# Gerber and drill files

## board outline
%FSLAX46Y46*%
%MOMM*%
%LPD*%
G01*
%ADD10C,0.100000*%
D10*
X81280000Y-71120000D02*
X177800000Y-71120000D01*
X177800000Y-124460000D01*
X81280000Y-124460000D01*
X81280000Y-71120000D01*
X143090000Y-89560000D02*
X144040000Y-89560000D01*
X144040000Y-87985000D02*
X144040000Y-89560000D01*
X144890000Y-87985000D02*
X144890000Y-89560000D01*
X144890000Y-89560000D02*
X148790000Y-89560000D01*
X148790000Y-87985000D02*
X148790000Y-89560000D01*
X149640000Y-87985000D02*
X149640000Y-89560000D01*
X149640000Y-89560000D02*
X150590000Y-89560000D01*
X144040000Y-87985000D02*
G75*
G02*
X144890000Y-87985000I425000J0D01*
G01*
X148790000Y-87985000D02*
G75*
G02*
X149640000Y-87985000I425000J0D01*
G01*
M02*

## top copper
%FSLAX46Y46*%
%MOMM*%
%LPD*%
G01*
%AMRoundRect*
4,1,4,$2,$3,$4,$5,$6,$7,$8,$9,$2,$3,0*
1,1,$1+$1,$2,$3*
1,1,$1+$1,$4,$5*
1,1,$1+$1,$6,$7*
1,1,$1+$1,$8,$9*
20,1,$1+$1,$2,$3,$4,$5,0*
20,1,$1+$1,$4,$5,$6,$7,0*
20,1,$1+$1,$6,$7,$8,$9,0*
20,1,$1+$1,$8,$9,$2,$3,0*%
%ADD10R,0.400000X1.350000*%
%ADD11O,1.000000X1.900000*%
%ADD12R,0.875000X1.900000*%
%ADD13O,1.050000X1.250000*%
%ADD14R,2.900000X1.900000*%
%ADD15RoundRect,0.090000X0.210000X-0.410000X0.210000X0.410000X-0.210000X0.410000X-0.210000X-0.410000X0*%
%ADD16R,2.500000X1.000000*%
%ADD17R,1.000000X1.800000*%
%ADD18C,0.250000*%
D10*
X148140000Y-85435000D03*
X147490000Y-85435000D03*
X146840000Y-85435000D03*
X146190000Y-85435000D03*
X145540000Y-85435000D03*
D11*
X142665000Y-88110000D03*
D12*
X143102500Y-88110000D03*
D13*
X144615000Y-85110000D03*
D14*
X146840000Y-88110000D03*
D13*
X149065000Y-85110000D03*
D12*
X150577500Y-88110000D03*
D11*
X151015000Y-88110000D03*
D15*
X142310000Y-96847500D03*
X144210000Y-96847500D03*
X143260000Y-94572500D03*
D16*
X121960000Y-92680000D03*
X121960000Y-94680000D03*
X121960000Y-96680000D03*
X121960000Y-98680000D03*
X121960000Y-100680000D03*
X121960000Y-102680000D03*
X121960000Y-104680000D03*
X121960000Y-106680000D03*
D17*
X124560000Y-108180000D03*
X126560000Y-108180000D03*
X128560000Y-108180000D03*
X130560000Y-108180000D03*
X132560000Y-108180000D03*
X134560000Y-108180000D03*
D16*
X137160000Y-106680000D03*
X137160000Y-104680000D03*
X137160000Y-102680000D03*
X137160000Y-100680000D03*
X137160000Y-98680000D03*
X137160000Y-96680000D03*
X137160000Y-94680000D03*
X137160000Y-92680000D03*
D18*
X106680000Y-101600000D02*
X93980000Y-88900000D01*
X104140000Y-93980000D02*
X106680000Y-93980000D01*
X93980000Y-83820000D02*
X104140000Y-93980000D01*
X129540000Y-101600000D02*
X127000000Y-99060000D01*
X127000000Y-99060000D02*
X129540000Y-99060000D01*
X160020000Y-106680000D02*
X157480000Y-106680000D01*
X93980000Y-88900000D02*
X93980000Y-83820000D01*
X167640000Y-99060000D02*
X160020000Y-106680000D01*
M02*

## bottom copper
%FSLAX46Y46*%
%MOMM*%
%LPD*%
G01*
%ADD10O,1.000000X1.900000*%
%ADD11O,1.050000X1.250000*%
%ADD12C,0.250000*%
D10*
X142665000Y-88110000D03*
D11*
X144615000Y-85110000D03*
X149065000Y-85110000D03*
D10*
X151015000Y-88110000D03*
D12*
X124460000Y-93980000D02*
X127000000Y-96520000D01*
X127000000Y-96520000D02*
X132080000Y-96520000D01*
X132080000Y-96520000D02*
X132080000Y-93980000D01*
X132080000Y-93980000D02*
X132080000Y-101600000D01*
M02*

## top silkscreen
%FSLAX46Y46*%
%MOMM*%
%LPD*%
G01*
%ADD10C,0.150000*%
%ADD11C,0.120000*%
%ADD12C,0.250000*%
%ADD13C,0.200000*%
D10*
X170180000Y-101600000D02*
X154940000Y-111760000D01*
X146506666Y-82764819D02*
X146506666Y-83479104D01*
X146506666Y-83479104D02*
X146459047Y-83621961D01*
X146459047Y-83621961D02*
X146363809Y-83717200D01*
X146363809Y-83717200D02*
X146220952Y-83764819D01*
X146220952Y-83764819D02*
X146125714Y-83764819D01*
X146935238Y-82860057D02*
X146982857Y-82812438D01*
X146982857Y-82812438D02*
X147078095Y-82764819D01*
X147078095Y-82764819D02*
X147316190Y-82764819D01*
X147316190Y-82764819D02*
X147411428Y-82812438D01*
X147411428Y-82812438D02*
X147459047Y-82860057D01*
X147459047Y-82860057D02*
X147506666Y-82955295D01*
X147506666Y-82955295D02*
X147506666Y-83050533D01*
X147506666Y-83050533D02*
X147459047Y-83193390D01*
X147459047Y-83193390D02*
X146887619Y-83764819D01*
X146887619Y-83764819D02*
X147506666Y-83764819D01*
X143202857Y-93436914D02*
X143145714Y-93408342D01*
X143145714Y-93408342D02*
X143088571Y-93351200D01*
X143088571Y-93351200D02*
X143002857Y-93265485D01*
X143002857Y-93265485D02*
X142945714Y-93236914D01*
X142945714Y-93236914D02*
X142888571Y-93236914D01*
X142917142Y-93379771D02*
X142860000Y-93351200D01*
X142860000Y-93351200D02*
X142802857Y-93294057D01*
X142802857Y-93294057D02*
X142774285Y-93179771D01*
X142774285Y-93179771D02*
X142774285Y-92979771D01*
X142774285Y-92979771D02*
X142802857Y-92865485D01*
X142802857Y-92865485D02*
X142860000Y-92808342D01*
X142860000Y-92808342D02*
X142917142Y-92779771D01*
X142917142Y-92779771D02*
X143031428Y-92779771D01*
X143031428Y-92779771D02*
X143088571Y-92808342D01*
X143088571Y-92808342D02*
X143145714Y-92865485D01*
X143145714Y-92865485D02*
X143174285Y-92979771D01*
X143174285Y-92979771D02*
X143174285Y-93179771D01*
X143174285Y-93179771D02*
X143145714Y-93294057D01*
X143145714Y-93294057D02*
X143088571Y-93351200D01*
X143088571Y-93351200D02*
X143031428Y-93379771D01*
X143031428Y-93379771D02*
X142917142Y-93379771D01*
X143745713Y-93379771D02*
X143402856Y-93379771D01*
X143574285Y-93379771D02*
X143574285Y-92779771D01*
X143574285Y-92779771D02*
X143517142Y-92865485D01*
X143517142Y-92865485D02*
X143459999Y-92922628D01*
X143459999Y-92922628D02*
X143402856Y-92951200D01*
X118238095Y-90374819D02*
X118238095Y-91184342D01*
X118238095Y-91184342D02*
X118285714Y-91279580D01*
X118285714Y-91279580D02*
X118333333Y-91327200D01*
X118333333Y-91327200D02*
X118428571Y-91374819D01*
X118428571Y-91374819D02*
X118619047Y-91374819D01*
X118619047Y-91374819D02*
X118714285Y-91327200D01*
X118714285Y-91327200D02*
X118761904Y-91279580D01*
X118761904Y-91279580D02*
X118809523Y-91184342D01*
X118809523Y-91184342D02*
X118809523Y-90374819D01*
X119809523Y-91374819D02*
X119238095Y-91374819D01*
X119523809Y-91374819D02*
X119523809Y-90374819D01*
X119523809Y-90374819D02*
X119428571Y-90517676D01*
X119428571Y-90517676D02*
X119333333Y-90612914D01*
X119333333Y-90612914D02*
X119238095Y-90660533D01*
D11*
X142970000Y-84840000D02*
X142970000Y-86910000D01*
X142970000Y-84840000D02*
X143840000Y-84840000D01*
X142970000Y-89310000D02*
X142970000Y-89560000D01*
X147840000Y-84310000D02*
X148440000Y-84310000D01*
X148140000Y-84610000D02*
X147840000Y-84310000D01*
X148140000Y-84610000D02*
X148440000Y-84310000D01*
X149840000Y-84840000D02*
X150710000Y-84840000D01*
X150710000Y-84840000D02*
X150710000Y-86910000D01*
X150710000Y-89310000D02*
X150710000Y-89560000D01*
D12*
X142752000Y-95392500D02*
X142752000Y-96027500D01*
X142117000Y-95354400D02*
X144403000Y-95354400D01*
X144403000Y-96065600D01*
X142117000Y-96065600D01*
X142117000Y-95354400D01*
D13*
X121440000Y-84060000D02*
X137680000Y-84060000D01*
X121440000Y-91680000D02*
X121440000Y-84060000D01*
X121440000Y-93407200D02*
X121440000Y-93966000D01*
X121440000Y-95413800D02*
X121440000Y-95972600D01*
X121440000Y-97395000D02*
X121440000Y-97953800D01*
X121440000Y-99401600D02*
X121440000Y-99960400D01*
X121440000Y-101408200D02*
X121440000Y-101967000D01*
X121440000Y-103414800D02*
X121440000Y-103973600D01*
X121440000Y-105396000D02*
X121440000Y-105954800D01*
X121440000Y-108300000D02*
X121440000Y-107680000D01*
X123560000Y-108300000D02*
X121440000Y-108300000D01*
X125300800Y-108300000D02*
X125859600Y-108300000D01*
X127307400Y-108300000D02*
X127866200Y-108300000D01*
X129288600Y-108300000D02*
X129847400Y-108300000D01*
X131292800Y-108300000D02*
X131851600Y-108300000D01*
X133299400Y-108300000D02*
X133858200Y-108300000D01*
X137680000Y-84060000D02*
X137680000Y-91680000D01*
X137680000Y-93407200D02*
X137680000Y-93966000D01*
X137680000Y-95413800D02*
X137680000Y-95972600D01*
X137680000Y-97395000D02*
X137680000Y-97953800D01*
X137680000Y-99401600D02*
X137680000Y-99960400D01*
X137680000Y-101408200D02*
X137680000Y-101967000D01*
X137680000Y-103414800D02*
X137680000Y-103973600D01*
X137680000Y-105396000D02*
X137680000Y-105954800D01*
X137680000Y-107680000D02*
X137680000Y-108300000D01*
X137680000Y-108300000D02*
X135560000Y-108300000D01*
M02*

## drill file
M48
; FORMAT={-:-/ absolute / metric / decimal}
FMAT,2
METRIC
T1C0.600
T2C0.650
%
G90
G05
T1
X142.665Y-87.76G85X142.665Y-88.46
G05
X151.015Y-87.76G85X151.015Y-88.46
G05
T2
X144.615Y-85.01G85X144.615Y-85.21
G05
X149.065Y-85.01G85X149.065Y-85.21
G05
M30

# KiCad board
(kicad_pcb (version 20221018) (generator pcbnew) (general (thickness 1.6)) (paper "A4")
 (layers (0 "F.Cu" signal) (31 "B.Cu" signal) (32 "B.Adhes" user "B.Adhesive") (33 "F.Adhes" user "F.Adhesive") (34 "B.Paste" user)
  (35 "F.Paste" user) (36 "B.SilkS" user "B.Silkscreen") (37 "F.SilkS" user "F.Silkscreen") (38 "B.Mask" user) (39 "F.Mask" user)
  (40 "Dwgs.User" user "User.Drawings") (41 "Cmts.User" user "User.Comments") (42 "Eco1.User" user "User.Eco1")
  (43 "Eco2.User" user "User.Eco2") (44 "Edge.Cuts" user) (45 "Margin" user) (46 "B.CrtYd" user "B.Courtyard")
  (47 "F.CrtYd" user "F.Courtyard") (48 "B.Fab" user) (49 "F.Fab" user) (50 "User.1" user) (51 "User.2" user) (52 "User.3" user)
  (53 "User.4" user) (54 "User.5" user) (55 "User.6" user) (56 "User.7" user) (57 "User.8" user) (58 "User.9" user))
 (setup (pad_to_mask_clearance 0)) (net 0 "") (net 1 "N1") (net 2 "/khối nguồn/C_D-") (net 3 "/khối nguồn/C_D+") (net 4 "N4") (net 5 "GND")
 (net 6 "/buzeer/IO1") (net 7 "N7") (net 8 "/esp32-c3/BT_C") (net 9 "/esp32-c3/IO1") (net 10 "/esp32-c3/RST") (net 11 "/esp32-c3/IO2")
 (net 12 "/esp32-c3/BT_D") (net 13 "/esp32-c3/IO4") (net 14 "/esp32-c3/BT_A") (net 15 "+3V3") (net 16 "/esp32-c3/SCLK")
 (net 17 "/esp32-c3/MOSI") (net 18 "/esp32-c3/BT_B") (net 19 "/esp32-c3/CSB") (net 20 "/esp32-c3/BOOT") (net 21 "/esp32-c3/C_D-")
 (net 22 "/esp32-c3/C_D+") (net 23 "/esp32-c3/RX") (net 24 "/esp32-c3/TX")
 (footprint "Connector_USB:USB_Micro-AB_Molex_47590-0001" (layer "F.Cu") (at 146.84 88.11)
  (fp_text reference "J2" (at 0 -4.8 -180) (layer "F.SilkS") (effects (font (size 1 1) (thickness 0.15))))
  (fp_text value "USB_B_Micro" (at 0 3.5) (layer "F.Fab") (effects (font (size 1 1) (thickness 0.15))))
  (fp_line (start -3.87 -3.27) (end -3.87 -1.2) (stroke (width 0.12) (type solid)) (layer "F.SilkS"))
  (fp_line (start -3.87 -3.27) (end -3 -3.27) (stroke (width 0.12) (type solid)) (layer "F.SilkS"))
  (fp_line (start -3.87 1.2) (end -3.87 1.45) (stroke (width 0.12) (type solid)) (layer "F.SilkS"))
  (fp_line (start 1 -3.8) (end 1.6 -3.8) (stroke (width 0.12) (type solid)) (layer "F.SilkS"))
  (fp_line (start 1.3 -3.5) (end 1 -3.8) (stroke (width 0.12) (type solid)) (layer "F.SilkS"))
  (fp_line (start 1.3 -3.5) (end 1.6 -3.8) (stroke (width 0.12) (type solid)) (layer "F.SilkS"))
  (fp_line (start 3 -3.27) (end 3.87 -3.27) (stroke (width 0.12) (type solid)) (layer "F.SilkS"))
  (fp_line (start 3.87 -3.27) (end 3.87 -1.2) (stroke (width 0.12) (type solid)) (layer "F.SilkS"))
  (fp_line (start 3.87 1.2) (end 3.87 1.45) (stroke (width 0.12) (type solid)) (layer "F.SilkS"))
  (fp_line (start -3.75 1.45) (end -2.8 1.45) (stroke (width 0.1) (type solid)) (layer "Edge.Cuts"))
  (fp_line (start -2.8 -0.125) (end -2.8 1.45) (stroke (width 0.1) (type solid)) (layer "Edge.Cuts"))
  (fp_line (start -1.95 -0.125) (end -1.95 1.45) (stroke (width 0.1) (type solid)) (layer "Edge.Cuts"))
  (fp_line (start -1.95 1.45) (end 1.95 1.45) (stroke (width 0.1) (type solid)) (layer "Edge.Cuts"))
  (fp_line (start 1.95 -0.125) (end 1.95 1.45) (stroke (width 0.1) (type solid)) (layer "Edge.Cuts"))
  (fp_line (start 2.8 -0.125) (end 2.8 1.45) (stroke (width 0.1) (type solid)) (layer "Edge.Cuts"))
  (fp_line (start 2.8 1.45) (end 3.75 1.45) (stroke (width 0.1) (type solid)) (layer "Edge.Cuts"))
  (fp_arc (start -2.8 -0.125) (mid -2.375 -0.55) (end -1.95 -0.125) (stroke (width 0.1) (type solid)) (layer "Edge.Cuts"))
  (fp_arc (start 1.95 -0.125) (mid 2.375 -0.55) (end 2.8 -0.125) (stroke (width 0.1) (type solid)) (layer "Edge.Cuts"))
  (pad "" smd rect (at -3.5 0) (size 0.3 0.85) (layers "F.Paste"))
  (pad "" smd rect (at 3.5 0) (size 0.3 0.85) (layers "F.Paste"))
  (pad "1" smd rect (at 1.3 -2.675) (size 0.4 1.35) (layers "F.Cu" "F.Paste" "F.Mask") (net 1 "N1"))
  (pad "2" smd rect (at 0.65 -2.675) (size 0.4 1.35) (layers "F.Cu" "F.Paste" "F.Mask") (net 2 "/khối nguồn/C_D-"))
  (pad "3" smd rect (at 0 -2.675) (size 0.4 1.35) (layers "F.Cu" "F.Paste" "F.Mask") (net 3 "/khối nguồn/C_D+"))
  (pad "4" smd rect (at -0.65 -2.675) (size 0.4 1.35) (layers "F.Cu" "F.Paste" "F.Mask") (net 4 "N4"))
  (pad "5" smd rect (at -1.3 -2.675) (size 0.4 1.35) (layers "F.Cu" "F.Paste" "F.Mask") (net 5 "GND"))
  (pad "6" thru_hole oval (at -4.175 0) (size 1 1.9) (drill oval 0.6 1.3) (layers "*.Cu" "*.Mask") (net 5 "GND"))
  (pad "6" smd rect (at -3.7375 0) (size 0.875 1.9) (layers "F.Cu" "F.Mask") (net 5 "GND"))
  (pad "6" thru_hole oval (at -2.225 -3) (size 1.05 1.25) (drill oval 0.65 0.85) (layers "*.Cu" "*.Mask") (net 5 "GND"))
  (pad "6" smd rect (at 0 0) (size 2.9 1.9) (layers "F.Cu" "F.Paste" "F.Mask") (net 5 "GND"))
  (pad "6" thru_hole oval (at 2.225 -3) (size 1.05 1.25) (drill oval 0.65 0.85) (layers "*.Cu" "*.Mask") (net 5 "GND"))
  (pad "6" smd rect (at 3.7375 0) (size 0.875 1.9) (layers "F.Cu" "F.Mask") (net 5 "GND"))
  (pad "6" thru_hole oval (at 4.175 0) (size 1 1.9) (drill oval 0.6 1.3) (layers "*.Cu" "*.Mask") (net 5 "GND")))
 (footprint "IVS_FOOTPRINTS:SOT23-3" (layer "F.Cu") (at 143.26 95.71)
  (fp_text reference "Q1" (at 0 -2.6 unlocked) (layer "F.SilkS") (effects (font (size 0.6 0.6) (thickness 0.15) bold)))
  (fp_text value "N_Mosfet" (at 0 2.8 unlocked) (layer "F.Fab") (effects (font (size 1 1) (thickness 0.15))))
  (fp_line (start -0.508 -0.3175) (end -0.508 0.3175) (stroke (width 0.25) (type default)) (layer "F.SilkS"))
  (fp_rect (start -1.143 -0.3556) (end 1.143 0.3556) (stroke (width 0.25) (type default)) (fill none) (layer "F.SilkS"))
  (pad "1" smd roundrect (at -0.95 1.1375 90) (size 1 0.6) (layers "F.Cu" "F.Paste" "F.Mask") (roundrect_rratio 0.15) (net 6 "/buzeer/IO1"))
  (pad "2" smd roundrect (at 0.95 1.1375 90) (size 1 0.6) (layers "F.Cu" "F.Paste" "F.Mask") (roundrect_rratio 0.15) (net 5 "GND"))
  (pad "3" smd roundrect (at 0 -1.1375 90) (size 1 0.6) (layers "F.Cu" "F.Paste" "F.Mask") (roundrect_rratio 0.15) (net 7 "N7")))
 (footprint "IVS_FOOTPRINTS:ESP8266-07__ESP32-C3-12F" (layer "F.Cu") (at 121.44 91.68)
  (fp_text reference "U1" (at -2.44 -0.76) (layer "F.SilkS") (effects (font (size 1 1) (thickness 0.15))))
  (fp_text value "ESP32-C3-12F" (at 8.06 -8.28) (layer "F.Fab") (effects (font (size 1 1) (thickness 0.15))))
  (fp_line (start 0 -7.62) (end 16.24 -7.62) (stroke (width 0.2) (type solid)) (layer "F.SilkS"))
  (fp_line (start 0 0) (end 0 -7.62) (stroke (width 0.2) (type solid)) (layer "F.SilkS"))
  (fp_line (start 0 1.7272) (end 0 2.286) (stroke (width 0.2) (type solid)) (layer "F.SilkS"))
  (fp_line (start 0 3.7338) (end 0 4.2926) (stroke (width 0.2) (type solid)) (layer "F.SilkS"))
  (fp_line (start 0 5.715) (end 0 6.2738) (stroke (width 0.2) (type solid)) (layer "F.SilkS"))
  (fp_line (start 0 7.7216) (end 0 8.2804) (stroke (width 0.2) (type solid)) (layer "F.SilkS"))
  (fp_line (start 0 9.7282) (end 0 10.287) (stroke (width 0.2) (type solid)) (layer "F.SilkS"))
  (fp_line (start 0 11.7348) (end 0 12.2936) (stroke (width 0.2) (type solid)) (layer "F.SilkS"))
  (fp_line (start 0 13.716) (end 0 14.2748) (stroke (width 0.2) (type solid)) (layer "F.SilkS"))
  (fp_line (start 0 16.62) (end 0 16) (stroke (width 0.2) (type solid)) (layer "F.SilkS"))
  (fp_line (start 2.12 16.62) (end 0 16.62) (stroke (width 0.2) (type solid)) (layer "F.SilkS"))
  (fp_line (start 3.8608 16.62) (end 4.4196 16.62) (stroke (width 0.2) (type solid)) (layer "F.SilkS"))
  (fp_line (start 5.8674 16.62) (end 6.4262 16.62) (stroke (width 0.2) (type solid)) (layer "F.SilkS"))
  (fp_line (start 7.8486 16.62) (end 8.4074 16.62) (stroke (width 0.2) (type solid)) (layer "F.SilkS"))
  (fp_line (start 9.8528 16.62) (end 10.4116 16.62) (stroke (width 0.2) (type solid)) (layer "F.SilkS"))
  (fp_line (start 11.8594 16.62) (end 12.4182 16.62) (stroke (width 0.2) (type solid)) (layer "F.SilkS"))
  (fp_line (start 16.24 -7.62) (end 16.24 0) (stroke (width 0.2) (type solid)) (layer "F.SilkS"))
  (fp_line (start 16.24 1.7272) (end 16.24 2.286) (stroke (width 0.2) (type solid)) (layer "F.SilkS"))
  (fp_line (start 16.24 3.7338) (end 16.24 4.2926) (stroke (width 0.2) (type solid)) (layer "F.SilkS"))
  (fp_line (start 16.24 5.715) (end 16.24 6.2738) (stroke (width 0.2) (type solid)) (layer "F.SilkS"))
  (fp_line (start 16.24 7.7216) (end 16.24 8.2804) (stroke (width 0.2) (type solid)) (layer "F.SilkS"))
  (fp_line (start 16.24 9.7282) (end 16.24 10.287) (stroke (width 0.2) (type solid)) (layer "F.SilkS"))
  (fp_line (start 16.24 11.7348) (end 16.24 12.2936) (stroke (width 0.2) (type solid)) (layer "F.SilkS"))
  (fp_line (start 16.24 13.716) (end 16.24 14.2748) (stroke (width 0.2) (type solid)) (layer "F.SilkS"))
  (fp_line (start 16.24 16) (end 16.24 16.62) (stroke (width 0.2) (type solid)) (layer "F.SilkS"))
  (fp_line (start 16.24 16.62) (end 14.12 16.62) (stroke (width 0.2) (type solid)) (layer "F.SilkS"))
  (pad "1" smd rect (at 0.52 1) (size 2.5 1) (layers "F.Cu" "F.Paste" "F.Mask") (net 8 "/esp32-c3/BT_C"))
  (pad "2" smd rect (at 0.52 3) (size 2.5 1) (layers "F.Cu" "F.Paste" "F.Mask") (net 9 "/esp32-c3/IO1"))
  (pad "3" smd rect (at 0.52 5) (size 2.5 1) (layers "F.Cu" "F.Paste" "F.Mask") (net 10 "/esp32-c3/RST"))
  (pad "4" smd rect (at 0.52 7) (size 2.5 1) (layers "F.Cu" "F.Paste" "F.Mask") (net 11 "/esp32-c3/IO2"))
  (pad "5" smd rect (at 0.52 9) (size 2.5 1) (layers "F.Cu" "F.Paste" "F.Mask") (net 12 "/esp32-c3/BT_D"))
  (pad "6" smd rect (at 0.52 11) (size 2.5 1) (layers "F.Cu" "F.Paste" "F.Mask") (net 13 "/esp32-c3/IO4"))
  (pad "7" smd rect (at 0.52 13) (size 2.5 1) (layers "F.Cu" "F.Paste" "F.Mask") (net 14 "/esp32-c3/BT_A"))
  (pad "8" smd rect (at 0.52 15) (size 2.5 1) (layers "F.Cu" "F.Paste" "F.Mask") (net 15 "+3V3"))
  (pad "9" smd rect (at 3.12 16.5) (size 1 1.8) (layers "F.Cu" "F.Paste" "F.Mask"))
  (pad "10" smd rect (at 5.12 16.5) (size 1 1.8) (layers "F.Cu" "F.Paste" "F.Mask"))
  (pad "11" smd rect (at 7.12 16.5) (size 1 1.8) (layers "F.Cu" "F.Paste" "F.Mask"))
  (pad "12" smd rect (at 9.12 16.5) (size 1 1.8) (layers "F.Cu" "F.Paste" "F.Mask") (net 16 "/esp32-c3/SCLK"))
  (pad "13" smd rect (at 11.12 16.5) (size 1 1.8) (layers "F.Cu" "F.Paste" "F.Mask") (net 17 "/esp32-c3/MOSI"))
  (pad "14" smd rect (at 13.12 16.5) (size 1 1.8) (layers "F.Cu" "F.Paste" "F.Mask"))
  (pad "15" smd rect (at 15.72 15) (size 2.5 1) (layers "F.Cu" "F.Paste" "F.Mask") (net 5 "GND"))
  (pad "16" smd rect (at 15.72 13) (size 2.5 1) (layers "F.Cu" "F.Paste" "F.Mask") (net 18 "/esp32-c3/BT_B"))
  (pad "17" smd rect (at 15.72 11) (size 2.5 1) (layers "F.Cu" "F.Paste" "F.Mask") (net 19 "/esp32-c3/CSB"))
  (pad "18" smd rect (at 15.72 9) (size 2.5 1) (layers "F.Cu" "F.Paste" "F.Mask") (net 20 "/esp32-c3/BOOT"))
  (pad "19" smd rect (at 15.72 7) (size 2.5 1) (layers "F.Cu" "F.Paste" "F.Mask") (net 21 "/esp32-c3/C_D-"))
  (pad "20" smd rect (at 15.72 5) (size 2.5 1) (layers "F.Cu" "F.Paste" "F.Mask") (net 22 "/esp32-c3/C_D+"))
  (pad "21" smd rect (at 15.72 3) (size 2.5 1) (layers "F.Cu" "F.Paste" "F.Mask") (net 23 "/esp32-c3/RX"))
  (pad "22" smd rect (at 15.72 1) (size 2.5 1) (layers "F.Cu" "F.Paste" "F.Mask") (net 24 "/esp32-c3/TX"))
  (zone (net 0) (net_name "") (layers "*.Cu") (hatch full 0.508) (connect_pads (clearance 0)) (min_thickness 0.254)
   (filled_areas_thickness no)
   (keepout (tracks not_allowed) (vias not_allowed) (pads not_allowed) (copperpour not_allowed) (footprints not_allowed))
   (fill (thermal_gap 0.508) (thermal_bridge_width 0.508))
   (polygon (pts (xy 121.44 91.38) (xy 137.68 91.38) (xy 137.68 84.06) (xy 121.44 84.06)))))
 (gr_line (start 170.18 101.6) (end 154.94 111.76) (stroke (width 0.15) (type default)) (layer "F.SilkS"))
 (gr_rect (start 81.28 71.12) (end 177.8 124.46) (stroke (width 0.1) (type default)) (fill none) (layer "Edge.Cuts"))
 (segment (start 106.68 101.6) (end 93.98 88.9) (width 0.25) (layer "F.Cu") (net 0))
 (segment (start 104.14 93.98) (end 106.68 93.98) (width 0.25) (layer "F.Cu") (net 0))
 (segment (start 93.98 83.82) (end 104.14 93.98) (width 0.25) (layer "F.Cu") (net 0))
 (segment (start 129.54 101.6) (end 127 99.06) (width 0.25) (layer "F.Cu") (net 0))
 (segment (start 127 99.06) (end 129.54 99.06) (width 0.25) (layer "F.Cu") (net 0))
 (segment (start 160.02 106.68) (end 157.48 106.68) (width 0.25) (layer "F.Cu") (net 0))
 (segment (start 93.98 88.9) (end 93.98 83.82) (width 0.25) (layer "F.Cu") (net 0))
 (segment (start 167.64 99.06) (end 160.02 106.68) (width 0.25) (layer "F.Cu") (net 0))
 (segment (start 124.46 93.98) (end 127 96.52) (width 0.25) (layer "B.Cu") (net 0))
 (segment (start 127 96.52) (end 132.08 96.52) (width 0.25) (layer "B.Cu") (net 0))
 (segment (start 132.08 96.52) (end 132.08 93.98) (width 0.25) (layer "B.Cu") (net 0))
 (segment (start 132.08 93.98) (end 132.08 101.6) (width 0.25) (layer "B.Cu") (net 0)))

